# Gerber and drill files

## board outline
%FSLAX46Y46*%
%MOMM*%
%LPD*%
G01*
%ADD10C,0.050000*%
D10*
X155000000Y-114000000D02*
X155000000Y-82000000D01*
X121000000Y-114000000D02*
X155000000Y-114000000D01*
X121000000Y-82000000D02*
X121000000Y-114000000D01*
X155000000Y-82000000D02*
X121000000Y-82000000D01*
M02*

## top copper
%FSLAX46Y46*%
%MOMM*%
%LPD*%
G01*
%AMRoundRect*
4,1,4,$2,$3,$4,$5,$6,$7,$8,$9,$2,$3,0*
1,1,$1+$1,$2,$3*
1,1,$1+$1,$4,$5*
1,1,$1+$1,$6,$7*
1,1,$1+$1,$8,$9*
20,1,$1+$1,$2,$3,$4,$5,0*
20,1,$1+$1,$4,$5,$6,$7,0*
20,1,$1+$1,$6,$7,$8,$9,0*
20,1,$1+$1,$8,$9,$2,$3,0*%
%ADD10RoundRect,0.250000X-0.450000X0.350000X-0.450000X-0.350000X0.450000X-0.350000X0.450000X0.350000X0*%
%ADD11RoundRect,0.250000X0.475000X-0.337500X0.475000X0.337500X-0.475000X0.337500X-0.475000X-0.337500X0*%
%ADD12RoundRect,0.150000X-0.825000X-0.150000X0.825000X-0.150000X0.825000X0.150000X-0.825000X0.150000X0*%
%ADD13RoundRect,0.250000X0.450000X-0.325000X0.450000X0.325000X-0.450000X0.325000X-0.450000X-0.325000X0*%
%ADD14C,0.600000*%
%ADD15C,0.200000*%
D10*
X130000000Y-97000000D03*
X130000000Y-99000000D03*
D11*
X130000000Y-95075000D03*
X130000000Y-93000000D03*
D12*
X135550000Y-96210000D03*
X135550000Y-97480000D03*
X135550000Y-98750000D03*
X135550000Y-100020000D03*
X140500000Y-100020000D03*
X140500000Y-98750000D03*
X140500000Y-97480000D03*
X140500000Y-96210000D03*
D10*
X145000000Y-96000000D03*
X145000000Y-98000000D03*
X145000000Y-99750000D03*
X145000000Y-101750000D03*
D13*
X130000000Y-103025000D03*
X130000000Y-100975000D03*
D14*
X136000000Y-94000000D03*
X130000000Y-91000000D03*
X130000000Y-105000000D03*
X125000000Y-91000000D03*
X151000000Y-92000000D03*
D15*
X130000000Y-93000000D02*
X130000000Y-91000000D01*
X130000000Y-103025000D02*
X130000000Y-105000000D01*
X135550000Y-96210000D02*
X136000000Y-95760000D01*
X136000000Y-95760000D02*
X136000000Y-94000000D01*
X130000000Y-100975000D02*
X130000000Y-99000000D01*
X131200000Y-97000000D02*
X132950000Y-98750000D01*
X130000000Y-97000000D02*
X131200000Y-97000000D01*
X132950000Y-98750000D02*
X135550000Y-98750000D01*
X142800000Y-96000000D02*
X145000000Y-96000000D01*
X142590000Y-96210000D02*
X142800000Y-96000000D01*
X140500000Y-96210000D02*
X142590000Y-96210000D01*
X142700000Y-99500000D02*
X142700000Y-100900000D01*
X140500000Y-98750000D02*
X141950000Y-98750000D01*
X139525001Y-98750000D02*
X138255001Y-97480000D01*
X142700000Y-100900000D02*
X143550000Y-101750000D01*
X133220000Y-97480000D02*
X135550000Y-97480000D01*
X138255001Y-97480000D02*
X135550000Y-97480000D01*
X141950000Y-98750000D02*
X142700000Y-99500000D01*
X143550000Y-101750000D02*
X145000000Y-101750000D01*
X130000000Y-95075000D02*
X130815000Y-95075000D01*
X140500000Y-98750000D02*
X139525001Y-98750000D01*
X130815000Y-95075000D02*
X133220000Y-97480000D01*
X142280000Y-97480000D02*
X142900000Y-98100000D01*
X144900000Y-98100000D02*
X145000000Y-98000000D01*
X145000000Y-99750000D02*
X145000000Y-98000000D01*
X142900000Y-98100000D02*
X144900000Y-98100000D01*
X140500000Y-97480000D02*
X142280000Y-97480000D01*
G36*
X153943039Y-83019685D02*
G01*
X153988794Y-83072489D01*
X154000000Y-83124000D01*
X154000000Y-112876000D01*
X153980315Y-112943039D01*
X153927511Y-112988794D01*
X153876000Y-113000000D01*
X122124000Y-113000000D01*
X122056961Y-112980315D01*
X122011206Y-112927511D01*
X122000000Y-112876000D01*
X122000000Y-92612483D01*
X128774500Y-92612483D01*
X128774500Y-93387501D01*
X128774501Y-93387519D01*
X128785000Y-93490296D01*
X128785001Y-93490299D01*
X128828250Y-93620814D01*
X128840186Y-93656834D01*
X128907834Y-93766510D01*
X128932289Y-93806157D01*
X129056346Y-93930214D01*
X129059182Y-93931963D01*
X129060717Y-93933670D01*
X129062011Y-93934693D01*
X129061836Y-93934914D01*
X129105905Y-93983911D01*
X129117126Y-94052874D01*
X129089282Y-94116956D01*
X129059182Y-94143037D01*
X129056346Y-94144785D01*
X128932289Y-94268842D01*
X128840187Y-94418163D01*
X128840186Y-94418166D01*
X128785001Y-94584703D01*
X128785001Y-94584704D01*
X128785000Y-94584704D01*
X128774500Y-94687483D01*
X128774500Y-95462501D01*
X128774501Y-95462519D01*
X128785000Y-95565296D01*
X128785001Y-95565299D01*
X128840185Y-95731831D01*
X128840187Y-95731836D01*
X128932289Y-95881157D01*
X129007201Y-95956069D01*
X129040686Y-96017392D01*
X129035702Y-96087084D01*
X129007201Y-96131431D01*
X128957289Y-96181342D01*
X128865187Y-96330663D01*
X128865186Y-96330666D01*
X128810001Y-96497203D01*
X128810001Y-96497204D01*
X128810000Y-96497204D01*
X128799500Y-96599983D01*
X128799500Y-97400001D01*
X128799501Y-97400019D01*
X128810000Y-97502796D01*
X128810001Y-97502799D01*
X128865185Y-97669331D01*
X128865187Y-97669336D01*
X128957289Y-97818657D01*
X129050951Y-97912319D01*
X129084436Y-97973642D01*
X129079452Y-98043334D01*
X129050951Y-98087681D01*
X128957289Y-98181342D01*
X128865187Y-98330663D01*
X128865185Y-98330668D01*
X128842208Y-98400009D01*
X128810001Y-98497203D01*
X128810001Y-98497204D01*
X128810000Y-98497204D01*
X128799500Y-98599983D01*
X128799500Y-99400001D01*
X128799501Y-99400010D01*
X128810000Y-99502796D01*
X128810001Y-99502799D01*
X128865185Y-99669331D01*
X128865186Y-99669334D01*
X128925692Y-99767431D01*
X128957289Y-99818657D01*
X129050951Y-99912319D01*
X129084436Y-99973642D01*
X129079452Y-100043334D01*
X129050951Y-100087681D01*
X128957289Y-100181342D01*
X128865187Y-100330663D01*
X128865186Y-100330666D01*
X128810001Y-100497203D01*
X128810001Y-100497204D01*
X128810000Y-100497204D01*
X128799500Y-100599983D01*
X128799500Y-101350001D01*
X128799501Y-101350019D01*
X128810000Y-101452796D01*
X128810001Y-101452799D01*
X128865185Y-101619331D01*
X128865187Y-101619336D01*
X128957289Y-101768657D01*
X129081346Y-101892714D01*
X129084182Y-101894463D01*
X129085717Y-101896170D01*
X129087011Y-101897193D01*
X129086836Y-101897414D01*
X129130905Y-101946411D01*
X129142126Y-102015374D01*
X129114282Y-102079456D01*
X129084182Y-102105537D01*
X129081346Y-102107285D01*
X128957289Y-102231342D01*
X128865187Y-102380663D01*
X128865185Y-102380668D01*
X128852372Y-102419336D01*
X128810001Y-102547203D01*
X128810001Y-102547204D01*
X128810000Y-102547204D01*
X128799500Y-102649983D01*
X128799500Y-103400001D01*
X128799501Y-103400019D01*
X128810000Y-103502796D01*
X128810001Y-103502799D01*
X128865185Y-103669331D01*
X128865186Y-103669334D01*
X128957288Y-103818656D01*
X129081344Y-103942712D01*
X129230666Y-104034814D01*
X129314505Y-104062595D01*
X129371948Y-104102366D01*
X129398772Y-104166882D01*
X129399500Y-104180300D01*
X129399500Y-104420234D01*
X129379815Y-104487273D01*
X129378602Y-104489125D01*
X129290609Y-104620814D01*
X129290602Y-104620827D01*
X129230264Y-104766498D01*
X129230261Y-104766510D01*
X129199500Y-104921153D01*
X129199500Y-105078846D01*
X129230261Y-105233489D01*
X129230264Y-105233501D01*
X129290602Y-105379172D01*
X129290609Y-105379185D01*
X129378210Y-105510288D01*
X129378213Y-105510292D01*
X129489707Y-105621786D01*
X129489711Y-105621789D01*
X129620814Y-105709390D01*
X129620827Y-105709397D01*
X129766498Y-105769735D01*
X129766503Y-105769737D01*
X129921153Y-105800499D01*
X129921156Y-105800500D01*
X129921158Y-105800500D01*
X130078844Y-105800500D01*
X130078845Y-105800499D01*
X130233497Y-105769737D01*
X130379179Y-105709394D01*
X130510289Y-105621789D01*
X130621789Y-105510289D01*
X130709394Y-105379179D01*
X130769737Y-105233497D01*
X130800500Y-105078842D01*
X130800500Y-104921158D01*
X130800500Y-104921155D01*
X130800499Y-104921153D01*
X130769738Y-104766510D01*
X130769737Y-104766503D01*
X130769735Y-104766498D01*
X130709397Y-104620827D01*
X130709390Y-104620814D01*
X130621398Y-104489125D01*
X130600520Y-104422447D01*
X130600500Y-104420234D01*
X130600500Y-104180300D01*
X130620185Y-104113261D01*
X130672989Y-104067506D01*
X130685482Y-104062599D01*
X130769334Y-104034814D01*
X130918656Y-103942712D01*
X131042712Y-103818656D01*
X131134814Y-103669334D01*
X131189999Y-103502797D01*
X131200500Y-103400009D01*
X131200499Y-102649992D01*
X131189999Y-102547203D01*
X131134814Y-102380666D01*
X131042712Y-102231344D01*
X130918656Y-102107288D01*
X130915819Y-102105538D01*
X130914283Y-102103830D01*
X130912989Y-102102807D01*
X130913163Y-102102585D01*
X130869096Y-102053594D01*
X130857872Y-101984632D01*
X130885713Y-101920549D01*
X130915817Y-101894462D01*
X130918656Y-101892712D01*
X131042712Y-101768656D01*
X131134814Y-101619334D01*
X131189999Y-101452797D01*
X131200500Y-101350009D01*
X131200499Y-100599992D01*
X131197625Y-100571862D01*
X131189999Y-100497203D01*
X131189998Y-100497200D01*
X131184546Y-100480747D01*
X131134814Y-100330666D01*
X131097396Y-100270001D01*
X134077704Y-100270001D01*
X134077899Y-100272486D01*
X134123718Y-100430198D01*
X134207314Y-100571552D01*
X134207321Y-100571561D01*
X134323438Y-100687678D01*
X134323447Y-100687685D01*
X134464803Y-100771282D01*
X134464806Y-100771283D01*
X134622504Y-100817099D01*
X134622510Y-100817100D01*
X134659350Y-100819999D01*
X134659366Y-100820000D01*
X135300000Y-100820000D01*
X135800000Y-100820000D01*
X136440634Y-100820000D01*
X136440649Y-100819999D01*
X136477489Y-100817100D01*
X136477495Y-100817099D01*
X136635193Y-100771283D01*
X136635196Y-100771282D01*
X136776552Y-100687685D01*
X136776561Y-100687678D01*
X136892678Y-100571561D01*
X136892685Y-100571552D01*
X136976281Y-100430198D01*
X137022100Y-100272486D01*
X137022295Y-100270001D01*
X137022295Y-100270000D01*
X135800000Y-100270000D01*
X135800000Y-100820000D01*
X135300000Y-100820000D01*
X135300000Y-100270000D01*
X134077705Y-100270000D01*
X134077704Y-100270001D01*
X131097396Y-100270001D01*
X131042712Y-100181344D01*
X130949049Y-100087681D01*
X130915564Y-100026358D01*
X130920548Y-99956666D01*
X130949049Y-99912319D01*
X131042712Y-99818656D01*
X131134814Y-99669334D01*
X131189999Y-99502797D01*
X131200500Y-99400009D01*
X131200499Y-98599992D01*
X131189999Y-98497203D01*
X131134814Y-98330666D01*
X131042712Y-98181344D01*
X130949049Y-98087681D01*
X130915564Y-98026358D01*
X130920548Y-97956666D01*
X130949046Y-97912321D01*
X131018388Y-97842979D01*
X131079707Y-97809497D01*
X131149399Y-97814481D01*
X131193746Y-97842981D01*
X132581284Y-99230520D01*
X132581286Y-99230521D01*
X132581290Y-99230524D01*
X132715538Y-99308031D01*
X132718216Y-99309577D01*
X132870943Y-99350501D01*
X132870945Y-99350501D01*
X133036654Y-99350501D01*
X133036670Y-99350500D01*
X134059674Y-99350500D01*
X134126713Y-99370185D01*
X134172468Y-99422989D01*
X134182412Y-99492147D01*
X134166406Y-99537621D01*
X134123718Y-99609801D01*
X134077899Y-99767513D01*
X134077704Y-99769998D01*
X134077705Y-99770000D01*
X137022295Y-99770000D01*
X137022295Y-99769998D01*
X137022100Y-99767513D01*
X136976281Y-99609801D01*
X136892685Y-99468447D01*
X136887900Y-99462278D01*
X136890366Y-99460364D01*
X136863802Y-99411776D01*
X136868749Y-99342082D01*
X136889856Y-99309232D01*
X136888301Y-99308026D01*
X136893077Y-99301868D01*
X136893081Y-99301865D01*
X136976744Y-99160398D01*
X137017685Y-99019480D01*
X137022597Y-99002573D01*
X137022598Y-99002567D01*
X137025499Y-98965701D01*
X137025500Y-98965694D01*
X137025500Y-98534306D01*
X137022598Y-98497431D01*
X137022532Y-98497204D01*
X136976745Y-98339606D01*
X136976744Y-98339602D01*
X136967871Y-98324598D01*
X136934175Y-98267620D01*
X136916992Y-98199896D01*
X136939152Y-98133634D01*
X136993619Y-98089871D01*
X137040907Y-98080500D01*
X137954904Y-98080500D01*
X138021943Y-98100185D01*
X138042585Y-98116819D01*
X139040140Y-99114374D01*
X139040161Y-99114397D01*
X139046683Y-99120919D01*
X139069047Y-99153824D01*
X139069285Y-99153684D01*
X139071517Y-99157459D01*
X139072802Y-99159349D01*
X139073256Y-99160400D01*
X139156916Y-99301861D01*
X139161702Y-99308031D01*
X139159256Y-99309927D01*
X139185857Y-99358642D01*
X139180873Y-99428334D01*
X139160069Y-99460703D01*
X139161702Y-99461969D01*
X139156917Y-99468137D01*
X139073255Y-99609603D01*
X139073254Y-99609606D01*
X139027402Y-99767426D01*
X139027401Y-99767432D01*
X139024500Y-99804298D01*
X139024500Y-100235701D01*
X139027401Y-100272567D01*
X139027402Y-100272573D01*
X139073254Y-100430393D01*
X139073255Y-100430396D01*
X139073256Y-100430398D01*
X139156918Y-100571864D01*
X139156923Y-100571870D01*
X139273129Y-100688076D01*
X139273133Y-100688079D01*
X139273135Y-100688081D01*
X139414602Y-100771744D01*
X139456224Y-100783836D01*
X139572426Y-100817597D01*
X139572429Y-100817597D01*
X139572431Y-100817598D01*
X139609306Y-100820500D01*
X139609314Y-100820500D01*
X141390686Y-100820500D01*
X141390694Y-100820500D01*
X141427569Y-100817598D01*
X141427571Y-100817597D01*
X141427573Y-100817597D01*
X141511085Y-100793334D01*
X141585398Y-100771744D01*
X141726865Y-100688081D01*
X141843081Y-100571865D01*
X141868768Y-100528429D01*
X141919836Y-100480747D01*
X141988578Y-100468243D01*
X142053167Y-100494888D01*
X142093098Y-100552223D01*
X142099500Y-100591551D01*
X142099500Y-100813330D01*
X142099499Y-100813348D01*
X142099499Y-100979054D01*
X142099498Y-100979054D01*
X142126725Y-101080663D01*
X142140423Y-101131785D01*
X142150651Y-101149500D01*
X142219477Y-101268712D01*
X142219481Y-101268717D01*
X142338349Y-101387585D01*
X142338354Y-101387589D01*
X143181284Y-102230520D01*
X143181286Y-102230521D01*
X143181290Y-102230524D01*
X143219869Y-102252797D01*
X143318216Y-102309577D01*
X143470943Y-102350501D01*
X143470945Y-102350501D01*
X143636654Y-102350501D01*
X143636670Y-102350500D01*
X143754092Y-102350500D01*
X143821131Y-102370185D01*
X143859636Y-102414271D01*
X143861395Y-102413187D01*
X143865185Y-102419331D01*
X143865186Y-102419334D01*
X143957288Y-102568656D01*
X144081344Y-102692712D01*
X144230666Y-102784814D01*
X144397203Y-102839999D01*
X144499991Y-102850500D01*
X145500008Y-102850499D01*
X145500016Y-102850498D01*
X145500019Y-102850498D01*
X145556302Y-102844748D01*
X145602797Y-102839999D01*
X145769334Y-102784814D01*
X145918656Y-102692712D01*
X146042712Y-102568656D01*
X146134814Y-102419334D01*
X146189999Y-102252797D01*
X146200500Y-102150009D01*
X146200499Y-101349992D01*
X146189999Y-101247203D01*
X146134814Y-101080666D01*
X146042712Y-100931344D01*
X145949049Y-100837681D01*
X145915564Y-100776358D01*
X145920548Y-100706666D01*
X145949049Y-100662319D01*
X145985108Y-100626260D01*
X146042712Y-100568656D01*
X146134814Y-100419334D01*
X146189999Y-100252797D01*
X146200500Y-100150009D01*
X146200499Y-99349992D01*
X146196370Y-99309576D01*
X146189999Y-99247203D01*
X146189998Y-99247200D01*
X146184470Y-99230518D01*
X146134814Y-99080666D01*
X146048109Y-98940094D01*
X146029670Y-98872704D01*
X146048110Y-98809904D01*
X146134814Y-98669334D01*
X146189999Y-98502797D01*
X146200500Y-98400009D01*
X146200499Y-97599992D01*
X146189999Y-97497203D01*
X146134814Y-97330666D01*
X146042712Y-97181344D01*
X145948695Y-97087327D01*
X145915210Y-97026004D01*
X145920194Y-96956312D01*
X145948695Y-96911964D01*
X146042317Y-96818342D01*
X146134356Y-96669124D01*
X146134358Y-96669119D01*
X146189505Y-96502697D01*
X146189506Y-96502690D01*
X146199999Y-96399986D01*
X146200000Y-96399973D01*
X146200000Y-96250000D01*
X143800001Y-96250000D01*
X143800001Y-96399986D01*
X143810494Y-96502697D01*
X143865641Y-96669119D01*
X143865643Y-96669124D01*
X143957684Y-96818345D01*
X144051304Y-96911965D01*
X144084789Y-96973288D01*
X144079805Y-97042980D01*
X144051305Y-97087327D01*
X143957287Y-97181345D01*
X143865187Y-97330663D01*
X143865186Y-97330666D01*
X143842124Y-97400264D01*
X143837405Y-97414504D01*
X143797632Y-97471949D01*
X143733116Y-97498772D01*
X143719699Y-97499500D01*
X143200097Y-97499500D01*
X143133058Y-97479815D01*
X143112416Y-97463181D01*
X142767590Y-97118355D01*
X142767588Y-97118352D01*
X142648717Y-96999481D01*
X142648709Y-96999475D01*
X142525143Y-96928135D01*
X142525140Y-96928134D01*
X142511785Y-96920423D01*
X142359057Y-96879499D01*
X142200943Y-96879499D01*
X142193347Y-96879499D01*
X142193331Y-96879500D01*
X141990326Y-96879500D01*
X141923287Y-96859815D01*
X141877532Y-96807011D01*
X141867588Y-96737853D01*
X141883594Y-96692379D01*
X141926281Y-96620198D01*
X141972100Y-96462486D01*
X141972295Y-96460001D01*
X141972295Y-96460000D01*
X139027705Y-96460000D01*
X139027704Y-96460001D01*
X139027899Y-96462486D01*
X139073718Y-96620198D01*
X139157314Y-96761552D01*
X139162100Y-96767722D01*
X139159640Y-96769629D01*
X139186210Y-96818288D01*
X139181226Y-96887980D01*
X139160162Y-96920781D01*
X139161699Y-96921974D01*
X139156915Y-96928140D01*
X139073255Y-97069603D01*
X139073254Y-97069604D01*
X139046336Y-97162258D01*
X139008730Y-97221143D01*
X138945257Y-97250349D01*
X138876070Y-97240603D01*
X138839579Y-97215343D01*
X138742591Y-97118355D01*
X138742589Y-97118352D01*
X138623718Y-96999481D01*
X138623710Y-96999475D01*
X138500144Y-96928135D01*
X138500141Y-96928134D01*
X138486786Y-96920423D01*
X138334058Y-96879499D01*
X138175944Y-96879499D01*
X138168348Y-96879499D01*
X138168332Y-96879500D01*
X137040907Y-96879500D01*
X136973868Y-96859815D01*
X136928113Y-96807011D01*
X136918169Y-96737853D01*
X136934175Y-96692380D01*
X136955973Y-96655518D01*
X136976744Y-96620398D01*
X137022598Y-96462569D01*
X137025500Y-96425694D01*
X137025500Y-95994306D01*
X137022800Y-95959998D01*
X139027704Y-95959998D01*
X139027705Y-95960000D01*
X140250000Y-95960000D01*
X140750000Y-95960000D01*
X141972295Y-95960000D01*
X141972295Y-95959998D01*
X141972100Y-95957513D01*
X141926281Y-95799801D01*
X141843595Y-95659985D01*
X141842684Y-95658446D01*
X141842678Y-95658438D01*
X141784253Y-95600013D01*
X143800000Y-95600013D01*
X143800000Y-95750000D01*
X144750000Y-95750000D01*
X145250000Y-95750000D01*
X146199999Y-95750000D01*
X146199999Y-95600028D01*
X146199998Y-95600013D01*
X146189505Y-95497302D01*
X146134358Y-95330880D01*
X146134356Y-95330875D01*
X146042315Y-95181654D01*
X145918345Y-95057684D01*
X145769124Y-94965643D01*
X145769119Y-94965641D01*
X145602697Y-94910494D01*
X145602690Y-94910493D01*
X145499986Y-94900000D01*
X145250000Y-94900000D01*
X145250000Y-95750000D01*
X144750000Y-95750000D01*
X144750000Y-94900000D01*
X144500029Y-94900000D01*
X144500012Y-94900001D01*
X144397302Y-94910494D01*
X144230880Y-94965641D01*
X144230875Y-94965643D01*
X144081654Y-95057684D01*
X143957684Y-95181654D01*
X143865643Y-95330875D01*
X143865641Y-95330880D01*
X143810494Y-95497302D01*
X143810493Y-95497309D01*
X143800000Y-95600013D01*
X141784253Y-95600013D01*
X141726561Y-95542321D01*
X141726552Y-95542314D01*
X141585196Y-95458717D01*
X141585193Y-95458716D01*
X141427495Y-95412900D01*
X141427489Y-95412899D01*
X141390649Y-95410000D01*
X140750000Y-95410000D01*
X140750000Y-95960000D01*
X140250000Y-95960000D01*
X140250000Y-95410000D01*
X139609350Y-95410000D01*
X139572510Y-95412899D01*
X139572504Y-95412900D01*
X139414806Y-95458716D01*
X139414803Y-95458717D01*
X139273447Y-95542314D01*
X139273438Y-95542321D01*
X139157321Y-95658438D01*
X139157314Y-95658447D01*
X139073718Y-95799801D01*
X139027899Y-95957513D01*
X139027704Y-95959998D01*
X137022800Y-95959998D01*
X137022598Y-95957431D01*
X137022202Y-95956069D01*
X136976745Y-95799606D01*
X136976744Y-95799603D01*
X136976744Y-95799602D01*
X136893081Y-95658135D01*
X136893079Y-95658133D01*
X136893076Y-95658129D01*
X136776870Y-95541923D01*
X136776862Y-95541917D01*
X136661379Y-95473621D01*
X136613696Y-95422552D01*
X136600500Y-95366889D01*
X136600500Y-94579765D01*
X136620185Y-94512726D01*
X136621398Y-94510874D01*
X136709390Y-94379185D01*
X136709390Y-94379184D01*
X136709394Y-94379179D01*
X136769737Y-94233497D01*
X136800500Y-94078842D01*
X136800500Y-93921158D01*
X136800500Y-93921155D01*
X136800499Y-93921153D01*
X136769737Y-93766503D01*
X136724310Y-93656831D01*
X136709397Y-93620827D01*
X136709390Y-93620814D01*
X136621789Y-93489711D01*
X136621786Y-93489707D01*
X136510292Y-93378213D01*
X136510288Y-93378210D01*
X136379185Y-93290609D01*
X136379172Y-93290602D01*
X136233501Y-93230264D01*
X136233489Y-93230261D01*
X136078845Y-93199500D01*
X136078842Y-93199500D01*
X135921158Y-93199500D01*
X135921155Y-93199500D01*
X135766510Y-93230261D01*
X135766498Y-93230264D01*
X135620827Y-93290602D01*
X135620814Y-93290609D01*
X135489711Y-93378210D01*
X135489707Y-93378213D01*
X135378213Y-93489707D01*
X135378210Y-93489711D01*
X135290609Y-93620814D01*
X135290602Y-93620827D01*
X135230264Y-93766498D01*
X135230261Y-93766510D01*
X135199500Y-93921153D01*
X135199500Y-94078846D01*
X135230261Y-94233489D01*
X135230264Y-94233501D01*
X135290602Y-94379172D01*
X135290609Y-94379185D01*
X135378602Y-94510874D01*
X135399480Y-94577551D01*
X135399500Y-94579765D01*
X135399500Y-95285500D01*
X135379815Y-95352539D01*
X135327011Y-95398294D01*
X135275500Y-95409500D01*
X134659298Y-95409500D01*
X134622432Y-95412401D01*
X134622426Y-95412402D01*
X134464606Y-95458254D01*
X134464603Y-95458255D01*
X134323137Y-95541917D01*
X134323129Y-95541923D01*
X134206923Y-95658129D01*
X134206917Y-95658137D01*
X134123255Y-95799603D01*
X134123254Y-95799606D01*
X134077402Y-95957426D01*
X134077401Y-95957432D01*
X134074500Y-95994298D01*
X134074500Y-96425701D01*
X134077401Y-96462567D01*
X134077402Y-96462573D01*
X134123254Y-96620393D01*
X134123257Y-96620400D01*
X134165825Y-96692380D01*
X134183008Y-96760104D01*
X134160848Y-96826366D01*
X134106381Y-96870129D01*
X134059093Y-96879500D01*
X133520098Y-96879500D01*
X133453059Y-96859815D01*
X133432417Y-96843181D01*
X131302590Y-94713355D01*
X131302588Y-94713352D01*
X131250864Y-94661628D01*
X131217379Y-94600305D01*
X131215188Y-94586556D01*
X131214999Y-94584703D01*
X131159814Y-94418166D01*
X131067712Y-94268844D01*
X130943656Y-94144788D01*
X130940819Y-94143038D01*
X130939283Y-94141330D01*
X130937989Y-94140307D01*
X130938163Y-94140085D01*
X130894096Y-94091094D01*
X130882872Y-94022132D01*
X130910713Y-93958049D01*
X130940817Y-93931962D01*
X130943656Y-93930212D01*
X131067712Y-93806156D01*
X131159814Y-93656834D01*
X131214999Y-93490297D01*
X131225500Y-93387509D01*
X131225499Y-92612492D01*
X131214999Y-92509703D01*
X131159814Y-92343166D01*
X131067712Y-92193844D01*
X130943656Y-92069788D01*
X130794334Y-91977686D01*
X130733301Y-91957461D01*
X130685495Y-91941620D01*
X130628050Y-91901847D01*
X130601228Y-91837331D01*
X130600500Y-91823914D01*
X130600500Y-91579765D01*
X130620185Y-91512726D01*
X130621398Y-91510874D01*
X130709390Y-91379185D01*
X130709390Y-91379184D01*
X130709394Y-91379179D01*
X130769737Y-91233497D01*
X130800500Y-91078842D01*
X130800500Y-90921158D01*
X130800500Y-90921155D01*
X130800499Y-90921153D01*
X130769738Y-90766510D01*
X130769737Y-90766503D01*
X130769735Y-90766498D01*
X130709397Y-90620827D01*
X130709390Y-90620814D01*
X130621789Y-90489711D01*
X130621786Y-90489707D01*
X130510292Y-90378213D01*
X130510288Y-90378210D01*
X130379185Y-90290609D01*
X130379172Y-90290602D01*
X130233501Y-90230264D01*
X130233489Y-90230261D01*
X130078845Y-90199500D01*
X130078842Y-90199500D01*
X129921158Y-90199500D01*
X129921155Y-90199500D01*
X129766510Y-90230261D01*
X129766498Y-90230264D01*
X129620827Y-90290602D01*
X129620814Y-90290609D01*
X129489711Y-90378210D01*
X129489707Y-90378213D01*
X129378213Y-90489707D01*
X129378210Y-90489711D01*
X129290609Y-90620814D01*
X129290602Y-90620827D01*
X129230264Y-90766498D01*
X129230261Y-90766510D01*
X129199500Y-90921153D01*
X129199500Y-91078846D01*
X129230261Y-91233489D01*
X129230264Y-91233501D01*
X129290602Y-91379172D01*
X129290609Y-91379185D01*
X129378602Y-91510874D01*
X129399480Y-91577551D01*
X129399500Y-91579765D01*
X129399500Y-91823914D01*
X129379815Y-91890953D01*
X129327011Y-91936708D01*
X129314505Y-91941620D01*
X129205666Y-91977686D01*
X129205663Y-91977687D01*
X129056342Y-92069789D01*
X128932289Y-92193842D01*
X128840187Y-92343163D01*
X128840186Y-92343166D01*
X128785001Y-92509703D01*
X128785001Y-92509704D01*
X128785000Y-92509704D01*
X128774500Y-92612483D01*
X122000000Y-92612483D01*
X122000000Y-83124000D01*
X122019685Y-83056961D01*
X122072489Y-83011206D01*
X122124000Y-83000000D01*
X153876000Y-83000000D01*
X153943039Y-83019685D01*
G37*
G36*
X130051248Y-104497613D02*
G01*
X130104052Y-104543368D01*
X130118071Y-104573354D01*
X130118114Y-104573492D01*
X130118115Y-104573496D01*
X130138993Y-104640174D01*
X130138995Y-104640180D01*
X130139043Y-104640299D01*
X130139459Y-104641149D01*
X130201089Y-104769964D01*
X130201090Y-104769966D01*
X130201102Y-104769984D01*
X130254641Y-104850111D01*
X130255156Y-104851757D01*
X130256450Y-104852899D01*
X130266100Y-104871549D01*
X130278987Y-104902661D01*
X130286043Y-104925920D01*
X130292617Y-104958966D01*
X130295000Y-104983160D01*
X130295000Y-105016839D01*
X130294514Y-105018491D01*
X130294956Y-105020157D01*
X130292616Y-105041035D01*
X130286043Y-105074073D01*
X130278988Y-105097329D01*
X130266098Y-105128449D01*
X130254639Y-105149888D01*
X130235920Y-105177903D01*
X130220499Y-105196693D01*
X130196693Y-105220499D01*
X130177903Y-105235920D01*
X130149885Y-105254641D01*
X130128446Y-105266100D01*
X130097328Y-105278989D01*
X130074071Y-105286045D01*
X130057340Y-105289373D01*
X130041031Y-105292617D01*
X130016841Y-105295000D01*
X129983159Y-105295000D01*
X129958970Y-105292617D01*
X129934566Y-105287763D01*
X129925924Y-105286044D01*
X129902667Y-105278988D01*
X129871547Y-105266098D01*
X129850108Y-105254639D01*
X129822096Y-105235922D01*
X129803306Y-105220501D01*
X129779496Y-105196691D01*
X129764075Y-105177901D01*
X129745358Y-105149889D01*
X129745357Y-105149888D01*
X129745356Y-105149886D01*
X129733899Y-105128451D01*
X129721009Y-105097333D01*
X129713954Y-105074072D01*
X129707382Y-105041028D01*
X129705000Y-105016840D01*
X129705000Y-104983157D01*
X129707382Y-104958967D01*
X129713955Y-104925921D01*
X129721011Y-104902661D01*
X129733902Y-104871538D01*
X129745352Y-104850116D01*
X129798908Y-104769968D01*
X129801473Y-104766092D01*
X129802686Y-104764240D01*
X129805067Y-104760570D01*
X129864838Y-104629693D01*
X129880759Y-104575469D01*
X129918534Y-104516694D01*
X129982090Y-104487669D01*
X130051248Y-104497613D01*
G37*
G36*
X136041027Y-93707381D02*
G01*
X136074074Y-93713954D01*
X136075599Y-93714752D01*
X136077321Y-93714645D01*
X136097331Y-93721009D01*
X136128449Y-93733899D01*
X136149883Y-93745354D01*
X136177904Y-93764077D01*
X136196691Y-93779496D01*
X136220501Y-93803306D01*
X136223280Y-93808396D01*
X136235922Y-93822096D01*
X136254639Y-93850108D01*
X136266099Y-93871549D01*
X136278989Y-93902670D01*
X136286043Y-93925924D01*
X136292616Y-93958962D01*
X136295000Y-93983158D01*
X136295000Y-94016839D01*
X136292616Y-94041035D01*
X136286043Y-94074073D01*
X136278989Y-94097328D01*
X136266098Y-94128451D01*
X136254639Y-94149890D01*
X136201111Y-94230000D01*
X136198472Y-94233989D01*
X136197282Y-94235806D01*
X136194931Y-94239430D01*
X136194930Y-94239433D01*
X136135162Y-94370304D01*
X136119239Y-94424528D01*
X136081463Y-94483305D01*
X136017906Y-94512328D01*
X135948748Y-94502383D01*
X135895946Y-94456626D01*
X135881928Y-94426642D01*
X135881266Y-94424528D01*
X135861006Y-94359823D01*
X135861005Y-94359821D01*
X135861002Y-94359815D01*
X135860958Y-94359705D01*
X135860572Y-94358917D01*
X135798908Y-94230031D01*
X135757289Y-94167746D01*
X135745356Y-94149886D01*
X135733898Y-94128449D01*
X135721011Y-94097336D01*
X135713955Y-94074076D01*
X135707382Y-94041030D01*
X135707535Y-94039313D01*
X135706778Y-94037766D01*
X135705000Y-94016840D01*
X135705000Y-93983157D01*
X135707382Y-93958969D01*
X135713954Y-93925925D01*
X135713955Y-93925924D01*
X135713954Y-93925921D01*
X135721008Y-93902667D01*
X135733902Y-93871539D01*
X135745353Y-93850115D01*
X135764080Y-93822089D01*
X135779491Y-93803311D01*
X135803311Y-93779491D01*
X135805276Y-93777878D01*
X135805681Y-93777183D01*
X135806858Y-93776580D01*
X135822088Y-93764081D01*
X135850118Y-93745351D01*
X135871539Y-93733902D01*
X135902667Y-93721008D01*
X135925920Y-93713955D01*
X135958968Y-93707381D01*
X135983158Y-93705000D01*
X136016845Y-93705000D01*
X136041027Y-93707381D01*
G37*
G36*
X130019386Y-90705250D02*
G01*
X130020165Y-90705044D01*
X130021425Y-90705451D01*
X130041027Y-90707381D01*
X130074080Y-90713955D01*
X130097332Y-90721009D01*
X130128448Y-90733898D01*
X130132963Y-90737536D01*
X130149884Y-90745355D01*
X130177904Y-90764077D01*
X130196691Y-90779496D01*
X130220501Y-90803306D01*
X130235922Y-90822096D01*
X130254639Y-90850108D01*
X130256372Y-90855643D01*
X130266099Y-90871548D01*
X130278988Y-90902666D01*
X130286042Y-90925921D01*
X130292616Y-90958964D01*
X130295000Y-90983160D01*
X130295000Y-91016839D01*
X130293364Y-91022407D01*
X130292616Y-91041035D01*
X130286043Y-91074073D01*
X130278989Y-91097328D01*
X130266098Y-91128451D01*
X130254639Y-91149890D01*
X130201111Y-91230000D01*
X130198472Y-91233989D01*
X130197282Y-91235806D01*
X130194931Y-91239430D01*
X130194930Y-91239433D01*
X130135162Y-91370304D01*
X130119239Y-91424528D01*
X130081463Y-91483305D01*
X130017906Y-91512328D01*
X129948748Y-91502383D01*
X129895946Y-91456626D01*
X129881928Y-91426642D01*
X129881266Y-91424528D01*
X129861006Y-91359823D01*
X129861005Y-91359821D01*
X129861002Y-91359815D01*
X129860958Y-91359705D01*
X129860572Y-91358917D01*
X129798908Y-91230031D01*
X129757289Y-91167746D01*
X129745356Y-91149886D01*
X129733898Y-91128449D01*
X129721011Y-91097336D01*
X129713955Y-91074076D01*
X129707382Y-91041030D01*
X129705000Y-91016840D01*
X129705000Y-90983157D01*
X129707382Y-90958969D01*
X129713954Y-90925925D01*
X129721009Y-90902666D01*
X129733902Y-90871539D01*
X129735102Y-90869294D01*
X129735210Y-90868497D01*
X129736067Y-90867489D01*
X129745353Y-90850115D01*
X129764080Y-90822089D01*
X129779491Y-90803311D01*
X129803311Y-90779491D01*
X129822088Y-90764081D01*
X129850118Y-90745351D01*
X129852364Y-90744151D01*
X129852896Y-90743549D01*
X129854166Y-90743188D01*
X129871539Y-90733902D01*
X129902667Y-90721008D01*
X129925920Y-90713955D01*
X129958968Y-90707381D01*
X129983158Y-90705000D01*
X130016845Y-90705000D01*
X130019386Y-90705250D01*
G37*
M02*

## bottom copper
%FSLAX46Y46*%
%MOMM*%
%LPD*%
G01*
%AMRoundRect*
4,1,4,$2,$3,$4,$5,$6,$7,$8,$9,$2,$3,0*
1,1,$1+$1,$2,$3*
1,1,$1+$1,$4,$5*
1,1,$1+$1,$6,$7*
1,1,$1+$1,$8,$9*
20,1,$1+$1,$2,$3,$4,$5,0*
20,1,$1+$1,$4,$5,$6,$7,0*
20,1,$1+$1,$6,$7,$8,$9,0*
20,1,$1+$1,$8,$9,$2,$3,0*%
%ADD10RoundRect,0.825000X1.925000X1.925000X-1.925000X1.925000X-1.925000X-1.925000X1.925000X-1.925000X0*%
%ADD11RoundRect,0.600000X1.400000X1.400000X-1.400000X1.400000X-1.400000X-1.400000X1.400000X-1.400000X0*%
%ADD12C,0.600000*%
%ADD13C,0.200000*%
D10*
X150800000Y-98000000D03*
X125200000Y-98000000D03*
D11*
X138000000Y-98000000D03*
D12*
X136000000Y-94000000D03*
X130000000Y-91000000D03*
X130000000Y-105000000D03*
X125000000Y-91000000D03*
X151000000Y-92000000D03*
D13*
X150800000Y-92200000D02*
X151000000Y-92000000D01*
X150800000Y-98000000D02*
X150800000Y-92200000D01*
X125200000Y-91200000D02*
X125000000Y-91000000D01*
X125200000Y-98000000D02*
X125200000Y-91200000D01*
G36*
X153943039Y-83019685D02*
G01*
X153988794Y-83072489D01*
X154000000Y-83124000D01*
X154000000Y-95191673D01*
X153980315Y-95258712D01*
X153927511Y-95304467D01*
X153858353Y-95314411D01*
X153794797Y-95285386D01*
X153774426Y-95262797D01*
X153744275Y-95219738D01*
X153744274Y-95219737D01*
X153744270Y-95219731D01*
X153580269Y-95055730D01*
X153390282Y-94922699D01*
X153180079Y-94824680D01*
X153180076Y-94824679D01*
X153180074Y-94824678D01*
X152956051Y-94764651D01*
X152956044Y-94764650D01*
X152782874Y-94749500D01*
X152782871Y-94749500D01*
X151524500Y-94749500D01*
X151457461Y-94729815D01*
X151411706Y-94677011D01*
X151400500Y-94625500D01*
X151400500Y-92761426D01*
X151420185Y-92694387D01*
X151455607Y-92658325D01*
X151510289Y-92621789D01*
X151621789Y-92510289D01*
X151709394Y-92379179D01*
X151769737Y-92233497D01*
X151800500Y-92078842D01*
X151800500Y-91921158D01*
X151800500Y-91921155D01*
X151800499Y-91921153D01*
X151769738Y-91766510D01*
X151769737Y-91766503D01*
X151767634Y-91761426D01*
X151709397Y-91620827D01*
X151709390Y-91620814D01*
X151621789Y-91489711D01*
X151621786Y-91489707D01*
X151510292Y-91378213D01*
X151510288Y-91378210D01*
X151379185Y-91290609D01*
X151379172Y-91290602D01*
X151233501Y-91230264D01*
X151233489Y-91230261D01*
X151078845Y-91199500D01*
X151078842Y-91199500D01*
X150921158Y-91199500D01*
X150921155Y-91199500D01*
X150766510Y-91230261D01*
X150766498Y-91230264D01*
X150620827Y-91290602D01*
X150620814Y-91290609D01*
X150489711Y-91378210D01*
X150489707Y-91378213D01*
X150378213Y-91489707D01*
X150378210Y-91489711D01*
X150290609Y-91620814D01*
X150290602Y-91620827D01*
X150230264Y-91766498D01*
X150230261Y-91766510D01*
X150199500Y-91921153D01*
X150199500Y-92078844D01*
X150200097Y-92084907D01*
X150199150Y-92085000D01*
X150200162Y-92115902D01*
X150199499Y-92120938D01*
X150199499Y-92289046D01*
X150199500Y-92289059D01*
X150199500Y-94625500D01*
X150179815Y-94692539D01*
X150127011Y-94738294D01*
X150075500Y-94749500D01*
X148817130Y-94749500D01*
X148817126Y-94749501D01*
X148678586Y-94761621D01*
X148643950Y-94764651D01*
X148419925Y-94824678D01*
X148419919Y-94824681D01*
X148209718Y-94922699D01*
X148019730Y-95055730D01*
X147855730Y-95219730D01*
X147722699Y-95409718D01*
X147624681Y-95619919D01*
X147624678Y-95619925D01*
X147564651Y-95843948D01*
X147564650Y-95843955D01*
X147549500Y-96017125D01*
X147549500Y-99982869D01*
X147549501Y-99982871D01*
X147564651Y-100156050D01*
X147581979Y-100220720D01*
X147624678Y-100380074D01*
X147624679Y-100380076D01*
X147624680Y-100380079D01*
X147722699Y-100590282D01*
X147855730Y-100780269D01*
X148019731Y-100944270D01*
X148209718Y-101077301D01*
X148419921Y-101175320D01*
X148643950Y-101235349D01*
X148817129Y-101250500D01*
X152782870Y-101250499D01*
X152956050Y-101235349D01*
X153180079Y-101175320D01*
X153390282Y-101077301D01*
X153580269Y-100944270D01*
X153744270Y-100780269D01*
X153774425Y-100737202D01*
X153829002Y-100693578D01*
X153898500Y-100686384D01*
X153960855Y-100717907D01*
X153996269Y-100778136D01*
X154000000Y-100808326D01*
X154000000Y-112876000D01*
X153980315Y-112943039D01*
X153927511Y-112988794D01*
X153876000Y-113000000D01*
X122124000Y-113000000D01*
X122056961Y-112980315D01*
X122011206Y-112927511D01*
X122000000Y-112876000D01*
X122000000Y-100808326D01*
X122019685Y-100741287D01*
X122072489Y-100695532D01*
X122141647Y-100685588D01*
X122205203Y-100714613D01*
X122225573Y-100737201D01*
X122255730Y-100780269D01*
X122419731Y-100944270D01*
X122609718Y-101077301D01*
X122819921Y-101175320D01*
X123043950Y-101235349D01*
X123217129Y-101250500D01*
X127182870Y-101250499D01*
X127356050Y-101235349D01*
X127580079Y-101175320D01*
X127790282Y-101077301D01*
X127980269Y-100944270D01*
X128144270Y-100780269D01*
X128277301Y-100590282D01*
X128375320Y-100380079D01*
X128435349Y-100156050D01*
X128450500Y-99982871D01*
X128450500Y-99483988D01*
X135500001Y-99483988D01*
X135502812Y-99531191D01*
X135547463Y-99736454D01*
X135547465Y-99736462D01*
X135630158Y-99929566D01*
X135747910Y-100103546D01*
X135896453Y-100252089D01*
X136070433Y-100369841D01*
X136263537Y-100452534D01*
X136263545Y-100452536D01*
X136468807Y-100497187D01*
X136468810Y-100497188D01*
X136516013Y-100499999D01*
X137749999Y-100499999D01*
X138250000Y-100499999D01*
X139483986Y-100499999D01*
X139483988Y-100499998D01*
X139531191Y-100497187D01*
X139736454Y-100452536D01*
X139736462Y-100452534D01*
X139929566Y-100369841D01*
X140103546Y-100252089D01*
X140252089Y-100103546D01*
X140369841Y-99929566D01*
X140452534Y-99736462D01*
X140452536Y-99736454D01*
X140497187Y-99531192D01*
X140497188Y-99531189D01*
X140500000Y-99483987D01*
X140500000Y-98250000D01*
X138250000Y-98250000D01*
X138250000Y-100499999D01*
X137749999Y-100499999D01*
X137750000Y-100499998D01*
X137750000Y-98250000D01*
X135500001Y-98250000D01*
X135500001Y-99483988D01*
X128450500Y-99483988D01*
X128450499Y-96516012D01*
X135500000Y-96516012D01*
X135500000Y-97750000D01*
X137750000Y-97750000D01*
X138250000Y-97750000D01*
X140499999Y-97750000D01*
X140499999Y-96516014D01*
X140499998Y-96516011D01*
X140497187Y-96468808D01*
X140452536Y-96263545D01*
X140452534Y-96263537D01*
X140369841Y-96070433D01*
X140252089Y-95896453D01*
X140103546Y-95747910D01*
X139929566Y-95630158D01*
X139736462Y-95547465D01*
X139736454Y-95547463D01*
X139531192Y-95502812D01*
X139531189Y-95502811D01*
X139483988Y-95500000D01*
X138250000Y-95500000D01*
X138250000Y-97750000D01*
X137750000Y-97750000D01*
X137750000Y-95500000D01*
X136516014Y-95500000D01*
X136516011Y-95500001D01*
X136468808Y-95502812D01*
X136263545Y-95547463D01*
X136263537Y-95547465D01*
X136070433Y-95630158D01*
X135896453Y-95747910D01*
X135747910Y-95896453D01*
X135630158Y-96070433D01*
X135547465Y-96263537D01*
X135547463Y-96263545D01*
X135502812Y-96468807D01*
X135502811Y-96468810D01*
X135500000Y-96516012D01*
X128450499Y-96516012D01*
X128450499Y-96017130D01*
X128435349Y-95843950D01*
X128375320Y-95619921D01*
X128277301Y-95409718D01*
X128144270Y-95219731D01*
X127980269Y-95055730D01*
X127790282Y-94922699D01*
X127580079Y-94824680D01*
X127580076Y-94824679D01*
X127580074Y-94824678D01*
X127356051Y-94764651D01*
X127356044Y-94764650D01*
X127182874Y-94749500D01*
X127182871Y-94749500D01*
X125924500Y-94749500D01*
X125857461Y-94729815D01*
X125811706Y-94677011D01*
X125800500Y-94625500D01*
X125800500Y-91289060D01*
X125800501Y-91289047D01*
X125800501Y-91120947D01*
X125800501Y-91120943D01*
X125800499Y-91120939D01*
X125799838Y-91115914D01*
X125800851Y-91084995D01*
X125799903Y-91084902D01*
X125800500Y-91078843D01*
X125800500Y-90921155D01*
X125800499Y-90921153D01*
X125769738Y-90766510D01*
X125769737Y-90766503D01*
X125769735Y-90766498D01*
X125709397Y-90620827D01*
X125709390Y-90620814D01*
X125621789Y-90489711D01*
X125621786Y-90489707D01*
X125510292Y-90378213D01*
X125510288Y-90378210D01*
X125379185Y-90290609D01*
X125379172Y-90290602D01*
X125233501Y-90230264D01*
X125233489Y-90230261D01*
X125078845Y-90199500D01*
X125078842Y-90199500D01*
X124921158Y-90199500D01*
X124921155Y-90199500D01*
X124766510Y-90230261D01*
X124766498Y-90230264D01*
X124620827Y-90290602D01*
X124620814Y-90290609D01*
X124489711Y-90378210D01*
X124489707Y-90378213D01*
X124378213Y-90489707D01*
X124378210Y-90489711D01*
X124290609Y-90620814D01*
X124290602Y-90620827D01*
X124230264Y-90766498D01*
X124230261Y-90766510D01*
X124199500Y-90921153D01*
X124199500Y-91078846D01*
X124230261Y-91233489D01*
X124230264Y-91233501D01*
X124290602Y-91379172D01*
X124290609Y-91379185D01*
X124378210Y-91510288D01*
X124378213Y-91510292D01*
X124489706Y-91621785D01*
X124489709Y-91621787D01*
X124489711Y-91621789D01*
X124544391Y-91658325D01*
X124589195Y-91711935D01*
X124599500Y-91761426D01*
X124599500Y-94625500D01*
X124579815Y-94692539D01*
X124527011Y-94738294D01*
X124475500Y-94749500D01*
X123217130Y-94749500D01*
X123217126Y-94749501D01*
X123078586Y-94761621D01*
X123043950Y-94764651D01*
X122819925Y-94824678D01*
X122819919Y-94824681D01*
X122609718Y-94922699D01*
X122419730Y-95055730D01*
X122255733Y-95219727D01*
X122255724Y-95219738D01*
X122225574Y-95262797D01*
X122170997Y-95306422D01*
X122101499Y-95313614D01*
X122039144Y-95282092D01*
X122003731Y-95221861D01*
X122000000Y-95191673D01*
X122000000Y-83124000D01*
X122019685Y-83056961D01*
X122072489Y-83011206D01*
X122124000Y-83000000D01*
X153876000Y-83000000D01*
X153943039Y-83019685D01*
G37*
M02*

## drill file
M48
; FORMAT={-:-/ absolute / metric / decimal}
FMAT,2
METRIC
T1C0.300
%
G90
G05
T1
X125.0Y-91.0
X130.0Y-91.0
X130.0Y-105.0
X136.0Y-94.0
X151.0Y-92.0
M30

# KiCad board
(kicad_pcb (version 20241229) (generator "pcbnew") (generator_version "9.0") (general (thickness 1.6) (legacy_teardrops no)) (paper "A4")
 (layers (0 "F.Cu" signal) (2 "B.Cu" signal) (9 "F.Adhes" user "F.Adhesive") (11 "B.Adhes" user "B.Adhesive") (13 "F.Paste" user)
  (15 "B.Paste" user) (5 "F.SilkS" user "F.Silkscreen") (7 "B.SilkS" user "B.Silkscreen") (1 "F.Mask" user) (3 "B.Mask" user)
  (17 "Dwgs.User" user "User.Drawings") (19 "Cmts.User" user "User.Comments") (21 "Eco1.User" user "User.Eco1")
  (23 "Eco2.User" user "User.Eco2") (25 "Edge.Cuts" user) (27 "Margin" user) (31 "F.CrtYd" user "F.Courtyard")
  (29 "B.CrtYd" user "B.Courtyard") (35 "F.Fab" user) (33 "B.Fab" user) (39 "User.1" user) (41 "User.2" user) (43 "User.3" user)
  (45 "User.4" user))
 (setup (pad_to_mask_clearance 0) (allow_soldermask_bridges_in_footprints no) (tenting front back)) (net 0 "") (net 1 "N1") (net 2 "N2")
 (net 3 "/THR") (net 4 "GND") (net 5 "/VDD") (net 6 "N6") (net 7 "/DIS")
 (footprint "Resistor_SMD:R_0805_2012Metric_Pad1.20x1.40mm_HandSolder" (layer "F.Cu") (at 130 98 -90)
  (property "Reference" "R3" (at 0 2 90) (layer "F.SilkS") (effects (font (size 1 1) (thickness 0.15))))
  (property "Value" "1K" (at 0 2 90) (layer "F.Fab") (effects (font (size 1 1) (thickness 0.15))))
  (pad "1" smd roundrect (at -1 0 270) (size 1.2 1.4) (layers "F.Cu" "F.Mask" "F.Paste") (roundrect_rratio 0.208333) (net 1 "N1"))
  (pad "2" smd roundrect (at 1 0 270) (size 1.2 1.4) (layers "F.Cu" "F.Mask" "F.Paste") (roundrect_rratio 0.208333) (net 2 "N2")))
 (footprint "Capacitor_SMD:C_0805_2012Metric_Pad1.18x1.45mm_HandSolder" (layer "F.Cu") (at 130 94.0375 90)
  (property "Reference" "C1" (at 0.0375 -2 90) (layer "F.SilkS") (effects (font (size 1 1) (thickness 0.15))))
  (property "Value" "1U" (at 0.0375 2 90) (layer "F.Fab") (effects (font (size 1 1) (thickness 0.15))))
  (pad "1" smd roundrect (at -1.0375 0 90) (size 1.175 1.45) (layers "F.Cu" "F.Mask" "F.Paste") (roundrect_rratio 0.212766) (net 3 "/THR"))
  (pad "2" smd roundrect (at 1.0375 0 90) (size 1.175 1.45) (layers "F.Cu" "F.Mask" "F.Paste") (roundrect_rratio 0.212766) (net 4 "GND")))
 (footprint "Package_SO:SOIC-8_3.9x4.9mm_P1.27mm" (layer "F.Cu") (at 138.025 98.115)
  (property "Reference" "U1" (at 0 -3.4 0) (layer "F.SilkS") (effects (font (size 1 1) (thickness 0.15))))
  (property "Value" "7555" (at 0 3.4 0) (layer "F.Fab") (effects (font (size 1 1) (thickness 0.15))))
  (pad "1" smd roundrect (at -2.475 -1.905) (size 1.95 0.6) (layers "F.Cu" "F.Mask" "F.Paste") (roundrect_rratio 0.25) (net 4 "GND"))
  (pad "2" smd roundrect (at -2.475 -0.635) (size 1.95 0.6) (layers "F.Cu" "F.Mask" "F.Paste") (roundrect_rratio 0.25) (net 3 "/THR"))
  (pad "3" smd roundrect (at -2.475 0.635) (size 1.95 0.6) (layers "F.Cu" "F.Mask" "F.Paste") (roundrect_rratio 0.25) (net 1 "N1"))
  (pad "4" smd roundrect (at -2.475 1.905) (size 1.95 0.6) (layers "F.Cu" "F.Mask" "F.Paste") (roundrect_rratio 0.25) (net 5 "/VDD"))
  (pad "5" smd roundrect (at 2.475 1.905) (size 1.95 0.6) (layers "F.Cu" "F.Mask" "F.Paste") (roundrect_rratio 0.25) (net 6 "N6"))
  (pad "6" smd roundrect (at 2.475 0.635) (size 1.95 0.6) (layers "F.Cu" "F.Mask" "F.Paste") (roundrect_rratio 0.25) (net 3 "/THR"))
  (pad "7" smd roundrect (at 2.475 -0.635) (size 1.95 0.6) (layers "F.Cu" "F.Mask" "F.Paste") (roundrect_rratio 0.25) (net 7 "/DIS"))
  (pad "8" smd roundrect (at 2.475 -1.905) (size 1.95 0.6) (layers "F.Cu" "F.Mask" "F.Paste") (roundrect_rratio 0.25) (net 5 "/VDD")))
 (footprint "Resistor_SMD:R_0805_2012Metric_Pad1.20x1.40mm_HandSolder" (layer "F.Cu") (at 145 97 -90)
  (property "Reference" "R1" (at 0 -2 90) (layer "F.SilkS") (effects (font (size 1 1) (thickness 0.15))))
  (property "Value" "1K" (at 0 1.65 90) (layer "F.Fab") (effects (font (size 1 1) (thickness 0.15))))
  (pad "1" smd roundrect (at -1 0 270) (size 1.2 1.4) (layers "F.Cu" "F.Mask" "F.Paste") (roundrect_rratio 0.208333) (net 5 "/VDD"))
  (pad "2" smd roundrect (at 1 0 270) (size 1.2 1.4) (layers "F.Cu" "F.Mask" "F.Paste") (roundrect_rratio 0.208333) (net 7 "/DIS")))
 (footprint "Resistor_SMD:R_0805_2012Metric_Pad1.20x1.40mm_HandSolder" (layer "F.Cu") (at 145 100.75 -90)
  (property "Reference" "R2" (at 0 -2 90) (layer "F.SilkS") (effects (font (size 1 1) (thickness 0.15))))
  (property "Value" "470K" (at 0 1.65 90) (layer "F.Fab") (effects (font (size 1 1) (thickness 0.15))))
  (pad "1" smd roundrect (at -1 0 270) (size 1.2 1.4) (layers "F.Cu" "F.Mask" "F.Paste") (roundrect_rratio 0.208333) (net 7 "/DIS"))
  (pad "2" smd roundrect (at 1 0 270) (size 1.2 1.4) (layers "F.Cu" "F.Mask" "F.Paste") (roundrect_rratio 0.208333) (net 3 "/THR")))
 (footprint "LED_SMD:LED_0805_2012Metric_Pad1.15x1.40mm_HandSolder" (layer "F.Cu") (at 130 102 90)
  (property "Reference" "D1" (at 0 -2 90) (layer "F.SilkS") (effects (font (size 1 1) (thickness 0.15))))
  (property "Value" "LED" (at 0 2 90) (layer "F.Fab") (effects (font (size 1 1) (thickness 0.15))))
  (pad "1" smd roundrect (at -1.025 0 90) (size 1.15 1.4) (layers "F.Cu" "F.Mask" "F.Paste") (roundrect_rratio 0.217391) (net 4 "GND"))
  (pad "2" smd roundrect (at 1.025 0 90) (size 1.15 1.4) (layers "F.Cu" "F.Mask" "F.Paste") (roundrect_rratio 0.217391) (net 2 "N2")))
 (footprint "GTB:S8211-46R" (layer "B.Cu") (at 138 98 180)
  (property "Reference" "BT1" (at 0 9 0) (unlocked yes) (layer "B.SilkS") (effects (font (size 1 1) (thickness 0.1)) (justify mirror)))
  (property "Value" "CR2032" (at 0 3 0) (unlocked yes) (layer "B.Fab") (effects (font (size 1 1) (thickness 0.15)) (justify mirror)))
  (pad "1" smd roundrect (at -12.8 0 180) (size 5.5 5.5) (layers "B.Cu" "B.Mask" "B.Paste") (roundrect_rratio 0.15) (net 5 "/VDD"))
  (pad "1" smd roundrect (at 12.8 0 180) (size 5.5 5.5) (layers "B.Cu" "B.Mask" "B.Paste") (roundrect_rratio 0.15) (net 5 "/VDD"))
  (pad "2" smd roundrect (at 0 0 180) (size 4 4) (layers "B.Cu" "B.Mask" "B.Paste") (roundrect_rratio 0.15) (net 4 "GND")))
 (gr_line (start 155 114) (end 155 82) (stroke (width 0.05) (type default)) (layer "Edge.Cuts"))
 (gr_line (start 121 114) (end 155 114) (stroke (width 0.05) (type default)) (layer "Edge.Cuts"))
 (gr_line (start 121 82) (end 121 114) (stroke (width 0.05) (type default)) (layer "Edge.Cuts"))
 (gr_line (start 155 82) (end 121 82) (stroke (width 0.05) (type default)) (layer "Edge.Cuts"))
 (segment (start 130 93) (end 130 91) (width 0.2) (layer "F.Cu") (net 4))
 (segment (start 130 103.025) (end 130 105) (width 0.2) (layer "F.Cu") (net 4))
 (segment (start 135.55 96.21) (end 136 95.76) (width 0.2) (layer "F.Cu") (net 4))
 (segment (start 136 95.76) (end 136 94) (width 0.2) (layer "F.Cu") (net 4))
 (via (at 136 94) (size 0.6) (drill 0.3) (layers "F.Cu" "B.Cu") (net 4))
 (via (at 130 91) (size 0.6) (drill 0.3) (layers "F.Cu" "B.Cu") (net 4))
 (via (at 130 105) (size 0.6) (drill 0.3) (layers "F.Cu" "B.Cu") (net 4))
 (segment (start 130 100.975) (end 130 99) (width 0.2) (layer "F.Cu") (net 2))
 (segment (start 131.2 97) (end 132.95 98.75) (width 0.2) (layer "F.Cu") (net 1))
 (segment (start 130 97) (end 131.2 97) (width 0.2) (layer "F.Cu") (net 1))
 (segment (start 132.95 98.75) (end 135.55 98.75) (width 0.2) (layer "F.Cu") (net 1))
 (segment (start 142.8 96) (end 145 96) (width 0.2) (layer "F.Cu") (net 5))
 (segment (start 142.59 96.21) (end 142.8 96) (width 0.2) (layer "F.Cu") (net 5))
 (segment (start 140.5 96.21) (end 142.59 96.21) (width 0.2) (layer "F.Cu") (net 5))
 (via (at 125 91) (size 0.6) (drill 0.3) (layers "F.Cu" "B.Cu") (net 5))
 (via (at 151 92) (size 0.6) (drill 0.3) (layers "F.Cu" "B.Cu") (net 5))
 (segment (start 150.8 92.2) (end 151 92) (width 0.2) (layer "B.Cu") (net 5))
 (segment (start 150.8 98) (end 150.8 92.2) (width 0.2) (layer "B.Cu") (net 5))
 (segment (start 125.2 91.2) (end 125 91) (width 0.2) (layer "B.Cu") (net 5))
 (segment (start 125.2 98) (end 125.2 91.2) (width 0.2) (layer "B.Cu") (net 5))
 (segment (start 142.7 99.5) (end 142.7 100.9) (width 0.2) (layer "F.Cu") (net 3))
 (segment (start 140.5 98.75) (end 141.95 98.75) (width 0.2) (layer "F.Cu") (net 3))
 (segment (start 139.525001 98.75) (end 138.255001 97.48) (width 0.2) (layer "F.Cu") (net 3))
 (segment (start 142.7 100.9) (end 143.55 101.75) (width 0.2) (layer "F.Cu") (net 3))
 (segment (start 133.22 97.48) (end 135.55 97.48) (width 0.2) (layer "F.Cu") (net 3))
 (segment (start 138.255001 97.48) (end 135.55 97.48) (width 0.2) (layer "F.Cu") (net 3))
 (segment (start 141.95 98.75) (end 142.7 99.5) (width 0.2) (layer "F.Cu") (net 3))
 (segment (start 143.55 101.75) (end 145 101.75) (width 0.2) (layer "F.Cu") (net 3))
 (segment (start 130 95.075) (end 130.815 95.075) (width 0.2) (layer "F.Cu") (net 3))
 (segment (start 140.5 98.75) (end 139.525001 98.75) (width 0.2) (layer "F.Cu") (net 3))
 (segment (start 130.815 95.075) (end 133.22 97.48) (width 0.2) (layer "F.Cu") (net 3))
 (segment (start 142.28 97.48) (end 142.9 98.1) (width 0.2) (layer "F.Cu") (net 7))
 (segment (start 144.9 98.1) (end 145 98) (width 0.2) (layer "F.Cu") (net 7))
 (segment (start 145 99.75) (end 145 98) (width 0.2) (layer "F.Cu") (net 7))
 (segment (start 142.9 98.1) (end 144.9 98.1) (width 0.2) (layer "F.Cu") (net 7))
 (segment (start 140.5 97.48) (end 142.28 97.48) (width 0.2) (layer "F.Cu") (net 7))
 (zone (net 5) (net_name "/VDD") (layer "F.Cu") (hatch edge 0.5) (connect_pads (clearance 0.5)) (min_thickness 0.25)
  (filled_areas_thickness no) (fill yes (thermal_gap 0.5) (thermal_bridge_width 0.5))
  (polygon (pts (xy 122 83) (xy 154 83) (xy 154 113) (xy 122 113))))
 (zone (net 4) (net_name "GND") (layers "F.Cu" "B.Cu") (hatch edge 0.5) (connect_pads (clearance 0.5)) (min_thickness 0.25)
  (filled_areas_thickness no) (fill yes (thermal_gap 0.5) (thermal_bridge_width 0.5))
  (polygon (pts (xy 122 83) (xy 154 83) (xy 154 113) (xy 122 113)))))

